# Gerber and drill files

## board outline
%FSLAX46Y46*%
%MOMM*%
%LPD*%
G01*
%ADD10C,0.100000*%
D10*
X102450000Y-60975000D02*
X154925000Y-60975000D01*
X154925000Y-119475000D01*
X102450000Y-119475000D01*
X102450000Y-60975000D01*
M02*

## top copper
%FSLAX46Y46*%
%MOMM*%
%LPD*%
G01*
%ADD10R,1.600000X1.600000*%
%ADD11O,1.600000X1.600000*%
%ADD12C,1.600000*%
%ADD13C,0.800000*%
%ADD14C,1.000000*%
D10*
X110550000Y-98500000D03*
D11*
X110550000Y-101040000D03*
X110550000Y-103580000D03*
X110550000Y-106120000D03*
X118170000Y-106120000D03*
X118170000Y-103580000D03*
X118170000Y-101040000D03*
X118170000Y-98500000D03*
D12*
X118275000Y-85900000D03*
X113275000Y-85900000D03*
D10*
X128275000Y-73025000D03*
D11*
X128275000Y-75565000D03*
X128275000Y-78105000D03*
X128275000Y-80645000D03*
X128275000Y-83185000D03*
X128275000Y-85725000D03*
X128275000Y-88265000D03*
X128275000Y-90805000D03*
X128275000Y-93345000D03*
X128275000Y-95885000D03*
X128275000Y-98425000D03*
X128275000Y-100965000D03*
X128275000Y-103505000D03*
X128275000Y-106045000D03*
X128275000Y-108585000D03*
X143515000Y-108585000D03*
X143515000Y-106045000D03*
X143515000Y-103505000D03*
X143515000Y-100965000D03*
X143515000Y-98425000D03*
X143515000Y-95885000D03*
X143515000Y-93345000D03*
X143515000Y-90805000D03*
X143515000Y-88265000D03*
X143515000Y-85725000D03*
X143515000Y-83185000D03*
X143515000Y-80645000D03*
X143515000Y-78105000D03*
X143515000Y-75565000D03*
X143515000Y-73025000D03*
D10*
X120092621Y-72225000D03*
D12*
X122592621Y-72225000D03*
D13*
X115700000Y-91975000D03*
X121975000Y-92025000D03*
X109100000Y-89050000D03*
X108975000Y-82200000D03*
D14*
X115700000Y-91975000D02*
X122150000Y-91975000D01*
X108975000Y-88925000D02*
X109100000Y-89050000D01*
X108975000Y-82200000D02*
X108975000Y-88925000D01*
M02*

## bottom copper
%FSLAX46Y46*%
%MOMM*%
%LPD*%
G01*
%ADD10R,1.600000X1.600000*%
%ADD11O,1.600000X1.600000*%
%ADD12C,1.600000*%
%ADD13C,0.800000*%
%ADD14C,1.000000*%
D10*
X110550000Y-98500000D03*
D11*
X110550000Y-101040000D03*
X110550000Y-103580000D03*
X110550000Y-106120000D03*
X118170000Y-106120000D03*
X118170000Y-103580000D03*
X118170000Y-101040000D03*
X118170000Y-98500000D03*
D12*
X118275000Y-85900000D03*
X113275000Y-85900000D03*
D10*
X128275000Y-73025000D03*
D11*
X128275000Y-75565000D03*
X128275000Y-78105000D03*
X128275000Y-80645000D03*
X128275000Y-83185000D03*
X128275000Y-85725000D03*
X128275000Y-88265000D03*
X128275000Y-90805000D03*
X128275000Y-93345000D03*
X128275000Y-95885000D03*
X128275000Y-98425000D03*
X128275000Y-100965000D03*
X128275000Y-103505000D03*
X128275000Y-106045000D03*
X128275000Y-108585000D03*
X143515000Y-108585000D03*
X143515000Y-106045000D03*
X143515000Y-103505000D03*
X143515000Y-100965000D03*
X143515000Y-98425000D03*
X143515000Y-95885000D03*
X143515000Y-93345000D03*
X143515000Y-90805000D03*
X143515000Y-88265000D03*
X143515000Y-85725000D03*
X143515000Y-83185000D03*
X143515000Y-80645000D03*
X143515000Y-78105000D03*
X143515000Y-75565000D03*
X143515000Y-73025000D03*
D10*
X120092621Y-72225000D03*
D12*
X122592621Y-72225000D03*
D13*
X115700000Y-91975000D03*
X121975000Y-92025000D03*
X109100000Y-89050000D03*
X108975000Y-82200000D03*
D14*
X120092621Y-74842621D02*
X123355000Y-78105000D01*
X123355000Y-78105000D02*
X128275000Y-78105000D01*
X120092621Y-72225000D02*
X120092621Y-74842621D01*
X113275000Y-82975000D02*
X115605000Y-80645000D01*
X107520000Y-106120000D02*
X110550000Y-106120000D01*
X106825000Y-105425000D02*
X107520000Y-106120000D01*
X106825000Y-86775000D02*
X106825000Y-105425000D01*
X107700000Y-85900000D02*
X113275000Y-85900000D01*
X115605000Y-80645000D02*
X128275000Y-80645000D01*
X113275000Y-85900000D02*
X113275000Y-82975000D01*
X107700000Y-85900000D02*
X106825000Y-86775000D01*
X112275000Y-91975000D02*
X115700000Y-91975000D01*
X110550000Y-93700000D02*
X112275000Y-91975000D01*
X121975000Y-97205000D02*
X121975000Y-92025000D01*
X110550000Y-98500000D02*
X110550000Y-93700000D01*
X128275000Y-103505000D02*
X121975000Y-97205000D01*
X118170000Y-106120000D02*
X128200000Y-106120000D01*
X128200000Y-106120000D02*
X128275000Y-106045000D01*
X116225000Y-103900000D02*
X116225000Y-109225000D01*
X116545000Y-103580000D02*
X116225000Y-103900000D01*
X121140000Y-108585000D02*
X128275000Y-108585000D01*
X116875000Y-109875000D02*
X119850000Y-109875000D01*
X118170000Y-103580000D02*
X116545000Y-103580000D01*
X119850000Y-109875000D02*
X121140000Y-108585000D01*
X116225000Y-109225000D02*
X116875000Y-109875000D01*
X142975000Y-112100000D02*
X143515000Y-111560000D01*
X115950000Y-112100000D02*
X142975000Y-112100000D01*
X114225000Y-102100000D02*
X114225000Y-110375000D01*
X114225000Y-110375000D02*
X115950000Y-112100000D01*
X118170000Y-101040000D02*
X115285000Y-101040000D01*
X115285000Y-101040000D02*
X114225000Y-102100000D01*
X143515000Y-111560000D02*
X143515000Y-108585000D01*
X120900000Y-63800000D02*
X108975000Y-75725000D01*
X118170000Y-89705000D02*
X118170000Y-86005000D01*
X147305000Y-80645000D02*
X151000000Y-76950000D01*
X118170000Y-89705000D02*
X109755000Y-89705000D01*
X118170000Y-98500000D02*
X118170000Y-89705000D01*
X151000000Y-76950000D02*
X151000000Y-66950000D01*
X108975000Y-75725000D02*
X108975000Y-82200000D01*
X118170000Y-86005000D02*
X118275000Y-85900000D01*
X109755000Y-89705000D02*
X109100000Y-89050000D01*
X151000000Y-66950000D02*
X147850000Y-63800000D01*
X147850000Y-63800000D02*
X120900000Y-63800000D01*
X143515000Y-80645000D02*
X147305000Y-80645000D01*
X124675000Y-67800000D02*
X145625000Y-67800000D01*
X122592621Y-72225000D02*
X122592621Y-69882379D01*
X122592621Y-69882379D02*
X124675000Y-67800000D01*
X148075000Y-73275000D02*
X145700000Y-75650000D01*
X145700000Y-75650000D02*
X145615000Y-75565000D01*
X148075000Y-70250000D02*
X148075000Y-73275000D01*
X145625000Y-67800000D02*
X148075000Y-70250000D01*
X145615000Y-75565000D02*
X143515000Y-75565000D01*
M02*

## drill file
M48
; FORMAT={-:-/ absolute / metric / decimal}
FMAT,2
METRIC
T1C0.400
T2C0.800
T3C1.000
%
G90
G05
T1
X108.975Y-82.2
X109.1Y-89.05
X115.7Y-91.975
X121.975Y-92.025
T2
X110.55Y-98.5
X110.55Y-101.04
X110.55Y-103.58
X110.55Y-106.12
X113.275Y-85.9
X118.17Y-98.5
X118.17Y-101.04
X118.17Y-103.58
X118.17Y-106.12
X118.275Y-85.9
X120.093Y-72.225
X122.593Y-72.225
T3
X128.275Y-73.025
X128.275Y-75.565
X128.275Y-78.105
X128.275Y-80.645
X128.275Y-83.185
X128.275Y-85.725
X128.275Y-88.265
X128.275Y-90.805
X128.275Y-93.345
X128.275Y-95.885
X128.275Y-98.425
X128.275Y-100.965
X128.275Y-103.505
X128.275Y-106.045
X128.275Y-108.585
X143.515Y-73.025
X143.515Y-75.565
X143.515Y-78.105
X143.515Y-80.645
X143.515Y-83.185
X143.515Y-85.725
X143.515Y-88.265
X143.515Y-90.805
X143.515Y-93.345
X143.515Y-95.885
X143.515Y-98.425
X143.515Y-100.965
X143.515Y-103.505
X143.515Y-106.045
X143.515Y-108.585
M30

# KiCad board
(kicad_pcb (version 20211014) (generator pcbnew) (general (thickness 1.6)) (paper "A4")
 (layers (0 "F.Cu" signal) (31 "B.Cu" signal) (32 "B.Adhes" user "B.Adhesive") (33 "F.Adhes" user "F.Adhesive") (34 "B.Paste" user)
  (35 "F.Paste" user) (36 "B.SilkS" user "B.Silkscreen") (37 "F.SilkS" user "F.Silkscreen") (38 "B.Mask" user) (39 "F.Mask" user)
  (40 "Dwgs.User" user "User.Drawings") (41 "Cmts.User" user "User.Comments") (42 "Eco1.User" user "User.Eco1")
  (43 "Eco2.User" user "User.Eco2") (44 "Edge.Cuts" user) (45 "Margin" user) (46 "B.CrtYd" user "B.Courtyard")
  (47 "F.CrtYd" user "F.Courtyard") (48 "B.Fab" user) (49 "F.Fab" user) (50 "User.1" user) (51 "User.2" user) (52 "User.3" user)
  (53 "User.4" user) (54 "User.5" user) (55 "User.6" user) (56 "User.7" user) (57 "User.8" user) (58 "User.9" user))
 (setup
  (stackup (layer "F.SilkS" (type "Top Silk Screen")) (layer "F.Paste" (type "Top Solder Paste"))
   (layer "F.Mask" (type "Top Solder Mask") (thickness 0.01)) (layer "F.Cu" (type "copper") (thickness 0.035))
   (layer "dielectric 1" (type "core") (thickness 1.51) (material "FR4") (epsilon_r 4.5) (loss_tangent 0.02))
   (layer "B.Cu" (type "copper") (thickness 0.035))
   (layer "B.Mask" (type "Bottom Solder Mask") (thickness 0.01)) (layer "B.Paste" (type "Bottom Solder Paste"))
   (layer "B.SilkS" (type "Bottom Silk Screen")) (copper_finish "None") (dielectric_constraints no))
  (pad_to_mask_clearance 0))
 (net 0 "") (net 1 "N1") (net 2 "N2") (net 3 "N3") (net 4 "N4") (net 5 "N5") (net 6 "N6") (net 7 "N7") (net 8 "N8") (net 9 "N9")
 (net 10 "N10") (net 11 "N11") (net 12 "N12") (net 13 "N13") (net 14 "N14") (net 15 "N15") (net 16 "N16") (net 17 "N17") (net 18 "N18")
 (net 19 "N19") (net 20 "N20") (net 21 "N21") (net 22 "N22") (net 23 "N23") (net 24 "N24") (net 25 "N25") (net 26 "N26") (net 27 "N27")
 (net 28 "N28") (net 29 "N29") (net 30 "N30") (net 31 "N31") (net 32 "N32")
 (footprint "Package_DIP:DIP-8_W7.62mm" (layer "F.Cu") (at 110.55 98.5)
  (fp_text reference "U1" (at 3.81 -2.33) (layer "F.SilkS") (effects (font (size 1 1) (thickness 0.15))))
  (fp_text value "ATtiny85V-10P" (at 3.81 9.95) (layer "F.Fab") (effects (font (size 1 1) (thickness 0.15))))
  (pad "1" thru_hole rect (at 0 0) (size 1.6 1.6) (drill 0.8) (layers *.Cu *.Mask) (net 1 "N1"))
  (pad "2" thru_hole oval (at 0 2.54) (size 1.6 1.6) (drill 0.8) (layers *.Cu *.Mask) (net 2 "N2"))
  (pad "3" thru_hole oval (at 0 5.08) (size 1.6 1.6) (drill 0.8) (layers *.Cu *.Mask) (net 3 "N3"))
  (pad "4" thru_hole oval (at 0 7.62) (size 1.6 1.6) (drill 0.8) (layers *.Cu *.Mask) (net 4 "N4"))
  (pad "5" thru_hole oval (at 7.62 7.62) (size 1.6 1.6) (drill 0.8) (layers *.Cu *.Mask) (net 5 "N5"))
  (pad "6" thru_hole oval (at 7.62 5.08) (size 1.6 1.6) (drill 0.8) (layers *.Cu *.Mask) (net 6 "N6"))
  (pad "7" thru_hole oval (at 7.62 2.54) (size 1.6 1.6) (drill 0.8) (layers *.Cu *.Mask) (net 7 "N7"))
  (pad "8" thru_hole oval (at 7.62 0) (size 1.6 1.6) (drill 0.8) (layers *.Cu *.Mask) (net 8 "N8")))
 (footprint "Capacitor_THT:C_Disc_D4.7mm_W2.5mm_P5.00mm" (layer "F.Cu") (at 118.275 85.9 180)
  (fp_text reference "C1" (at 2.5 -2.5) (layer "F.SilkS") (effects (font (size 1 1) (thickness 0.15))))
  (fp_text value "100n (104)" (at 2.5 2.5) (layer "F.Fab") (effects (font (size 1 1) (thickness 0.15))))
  (pad "1" thru_hole circle (at 0 0 180) (size 1.6 1.6) (drill 0.8) (layers *.Cu *.Mask) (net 8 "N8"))
  (pad "2" thru_hole circle (at 5 0 180) (size 1.6 1.6) (drill 0.8) (layers *.Cu *.Mask) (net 4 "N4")))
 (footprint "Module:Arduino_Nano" (layer "F.Cu") (at 128.275 73.025)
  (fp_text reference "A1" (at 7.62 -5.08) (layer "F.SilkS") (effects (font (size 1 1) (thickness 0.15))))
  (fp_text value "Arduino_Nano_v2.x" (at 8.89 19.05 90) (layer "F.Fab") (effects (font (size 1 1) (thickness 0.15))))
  (pad "1" thru_hole rect (at 0 0) (size 1.6 1.6) (drill 1) (layers *.Cu *.Mask) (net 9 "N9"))
  (pad "2" thru_hole oval (at 0 2.54) (size 1.6 1.6) (drill 1) (layers *.Cu *.Mask) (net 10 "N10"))
  (pad "3" thru_hole oval (at 0 5.08) (size 1.6 1.6) (drill 1) (layers *.Cu *.Mask) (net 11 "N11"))
  (pad "4" thru_hole oval (at 0 7.62) (size 1.6 1.6) (drill 1) (layers *.Cu *.Mask) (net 4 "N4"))
  (pad "5" thru_hole oval (at 0 10.16) (size 1.6 1.6) (drill 1) (layers *.Cu *.Mask) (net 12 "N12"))
  (pad "6" thru_hole oval (at 0 12.7) (size 1.6 1.6) (drill 1) (layers *.Cu *.Mask) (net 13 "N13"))
  (pad "7" thru_hole oval (at 0 15.24) (size 1.6 1.6) (drill 1) (layers *.Cu *.Mask) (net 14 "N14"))
  (pad "8" thru_hole oval (at 0 17.78) (size 1.6 1.6) (drill 1) (layers *.Cu *.Mask) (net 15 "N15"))
  (pad "9" thru_hole oval (at 0 20.32) (size 1.6 1.6) (drill 1) (layers *.Cu *.Mask) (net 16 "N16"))
  (pad "10" thru_hole oval (at 0 22.86) (size 1.6 1.6) (drill 1) (layers *.Cu *.Mask) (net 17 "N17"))
  (pad "11" thru_hole oval (at 0 25.4) (size 1.6 1.6) (drill 1) (layers *.Cu *.Mask) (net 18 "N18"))
  (pad "12" thru_hole oval (at 0 27.94) (size 1.6 1.6) (drill 1) (layers *.Cu *.Mask) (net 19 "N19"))
  (pad "13" thru_hole oval (at 0 30.48) (size 1.6 1.6) (drill 1) (layers *.Cu *.Mask) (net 1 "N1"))
  (pad "14" thru_hole oval (at 0 33.02) (size 1.6 1.6) (drill 1) (layers *.Cu *.Mask) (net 5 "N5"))
  (pad "15" thru_hole oval (at 0 35.56) (size 1.6 1.6) (drill 1) (layers *.Cu *.Mask) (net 6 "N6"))
  (pad "16" thru_hole oval (at 15.24 35.56) (size 1.6 1.6) (drill 1) (layers *.Cu *.Mask) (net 7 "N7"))
  (pad "17" thru_hole oval (at 15.24 33.02) (size 1.6 1.6) (drill 1) (layers *.Cu *.Mask) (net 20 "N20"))
  (pad "18" thru_hole oval (at 15.24 30.48) (size 1.6 1.6) (drill 1) (layers *.Cu *.Mask) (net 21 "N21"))
  (pad "19" thru_hole oval (at 15.24 27.94) (size 1.6 1.6) (drill 1) (layers *.Cu *.Mask) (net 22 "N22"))
  (pad "20" thru_hole oval (at 15.24 25.4) (size 1.6 1.6) (drill 1) (layers *.Cu *.Mask) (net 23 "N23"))
  (pad "21" thru_hole oval (at 15.24 22.86) (size 1.6 1.6) (drill 1) (layers *.Cu *.Mask) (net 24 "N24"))
  (pad "22" thru_hole oval (at 15.24 20.32) (size 1.6 1.6) (drill 1) (layers *.Cu *.Mask) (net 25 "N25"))
  (pad "23" thru_hole oval (at 15.24 17.78) (size 1.6 1.6) (drill 1) (layers *.Cu *.Mask) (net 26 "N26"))
  (pad "24" thru_hole oval (at 15.24 15.24) (size 1.6 1.6) (drill 1) (layers *.Cu *.Mask) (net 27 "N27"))
  (pad "25" thru_hole oval (at 15.24 12.7) (size 1.6 1.6) (drill 1) (layers *.Cu *.Mask) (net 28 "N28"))
  (pad "26" thru_hole oval (at 15.24 10.16) (size 1.6 1.6) (drill 1) (layers *.Cu *.Mask) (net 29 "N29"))
  (pad "27" thru_hole oval (at 15.24 7.62) (size 1.6 1.6) (drill 1) (layers *.Cu *.Mask) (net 8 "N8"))
  (pad "28" thru_hole oval (at 15.24 5.08) (size 1.6 1.6) (drill 1) (layers *.Cu *.Mask) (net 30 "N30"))
  (pad "29" thru_hole oval (at 15.24 2.54) (size 1.6 1.6) (drill 1) (layers *.Cu *.Mask) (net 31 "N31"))
  (pad "30" thru_hole oval (at 15.24 0) (size 1.6 1.6) (drill 1) (layers *.Cu *.Mask) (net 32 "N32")))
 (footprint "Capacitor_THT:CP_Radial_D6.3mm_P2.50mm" (layer "F.Cu") (at 120.092621 72.225)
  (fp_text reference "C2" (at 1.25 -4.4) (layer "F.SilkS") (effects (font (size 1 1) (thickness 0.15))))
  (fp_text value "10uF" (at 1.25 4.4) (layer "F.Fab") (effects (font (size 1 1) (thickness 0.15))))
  (pad "1" thru_hole rect (at 0 0) (size 1.6 1.6) (drill 0.8) (layers *.Cu *.Mask) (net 11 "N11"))
  (pad "2" thru_hole circle (at 2.5 0) (size 1.6 1.6) (drill 0.8) (layers *.Cu *.Mask) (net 31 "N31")))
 (gr_rect (start 102.45 60.975) (end 154.925 119.475) (layer "Edge.Cuts") (width 0.1) (fill none))
 (segment (start 120.092621 74.842621) (end 123.355 78.105) (width 1) (layer "B.Cu") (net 11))
 (segment (start 123.355 78.105) (end 128.275 78.105) (width 1) (layer "B.Cu") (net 11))
 (segment (start 120.092621 72.225) (end 120.092621 74.842621) (width 1) (layer "B.Cu") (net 11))
 (segment (start 113.275 82.975) (end 115.605 80.645) (width 1) (layer "B.Cu") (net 4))
 (segment (start 107.52 106.12) (end 110.55 106.12) (width 1) (layer "B.Cu") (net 4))
 (segment (start 106.825 105.425) (end 107.52 106.12) (width 1) (layer "B.Cu") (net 4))
 (segment (start 106.825 86.775) (end 106.825 105.425) (width 1) (layer "B.Cu") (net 4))
 (segment (start 107.7 85.9) (end 113.275 85.9) (width 1) (layer "B.Cu") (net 4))
 (segment (start 115.605 80.645) (end 128.275 80.645) (width 1) (layer "B.Cu") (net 4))
 (segment (start 113.275 85.9) (end 113.275 82.975) (width 1) (layer "B.Cu") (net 4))
 (segment (start 107.7 85.9) (end 106.825 86.775) (width 1) (layer "B.Cu") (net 4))
 (segment (start 115.7 91.975) (end 122.15 91.975) (width 1) (layer "F.Cu") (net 1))
 (via (at 115.7 91.975) (size 0.8) (drill 0.4) (layers "F.Cu" "B.Cu") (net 1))
 (via (at 121.975 92.025) (size 0.8) (drill 0.4) (layers "F.Cu" "B.Cu") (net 1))
 (segment (start 112.275 91.975) (end 115.7 91.975) (width 1) (layer "B.Cu") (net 1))
 (segment (start 110.55 93.7) (end 112.275 91.975) (width 1) (layer "B.Cu") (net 1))
 (segment (start 121.975 97.205) (end 121.975 92.025) (width 1) (layer "B.Cu") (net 1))
 (segment (start 110.55 98.5) (end 110.55 93.7) (width 1) (layer "B.Cu") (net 1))
 (segment (start 128.275 103.505) (end 121.975 97.205) (width 1) (layer "B.Cu") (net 1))
 (segment (start 118.17 106.12) (end 128.2 106.12) (width 1) (layer "B.Cu") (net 5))
 (segment (start 128.2 106.12) (end 128.275 106.045) (width 1) (layer "B.Cu") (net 5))
 (segment (start 116.225 103.9) (end 116.225 109.225) (width 1) (layer "B.Cu") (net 6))
 (segment (start 116.545 103.58) (end 116.225 103.9) (width 1) (layer "B.Cu") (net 6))
 (segment (start 121.14 108.585) (end 128.275 108.585) (width 1) (layer "B.Cu") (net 6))
 (segment (start 116.875 109.875) (end 119.85 109.875) (width 1) (layer "B.Cu") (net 6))
 (segment (start 118.17 103.58) (end 116.545 103.58) (width 1) (layer "B.Cu") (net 6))
 (segment (start 119.85 109.875) (end 121.14 108.585) (width 1) (layer "B.Cu") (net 6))
 (segment (start 116.225 109.225) (end 116.875 109.875) (width 1) (layer "B.Cu") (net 6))
 (segment (start 142.975 112.1) (end 143.515 111.56) (width 1) (layer "B.Cu") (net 7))
 (segment (start 115.95 112.1) (end 142.975 112.1) (width 1) (layer "B.Cu") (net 7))
 (segment (start 114.225 102.1) (end 114.225 110.375) (width 1) (layer "B.Cu") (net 7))
 (segment (start 114.225 110.375) (end 115.95 112.1) (width 1) (layer "B.Cu") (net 7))
 (segment (start 118.17 101.04) (end 115.285 101.04) (width 1) (layer "B.Cu") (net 7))
 (segment (start 115.285 101.04) (end 114.225 102.1) (width 1) (layer "B.Cu") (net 7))
 (segment (start 143.515 111.56) (end 143.515 108.585) (width 1) (layer "B.Cu") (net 7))
 (segment (start 108.975 88.925) (end 109.1 89.05) (width 1) (layer "F.Cu") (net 8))
 (segment (start 108.975 82.2) (end 108.975 88.925) (width 1) (layer "F.Cu") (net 8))
 (via (at 109.1 89.05) (size 0.8) (drill 0.4) (layers "F.Cu" "B.Cu") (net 8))
 (via (at 108.975 82.2) (size 0.8) (drill 0.4) (layers "F.Cu" "B.Cu") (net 8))
 (segment (start 120.9 63.8) (end 108.975 75.725) (width 1) (layer "B.Cu") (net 8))
 (segment (start 118.17 89.705) (end 118.17 86.005) (width 1) (layer "B.Cu") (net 8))
 (segment (start 147.305 80.645) (end 151 76.95) (width 1) (layer "B.Cu") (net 8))
 (segment (start 118.17 89.705) (end 109.755 89.705) (width 1) (layer "B.Cu") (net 8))
 (segment (start 118.17 98.5) (end 118.17 89.705) (width 1) (layer "B.Cu") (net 8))
 (segment (start 151 76.95) (end 151 66.95) (width 1) (layer "B.Cu") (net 8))
 (segment (start 108.975 75.725) (end 108.975 82.2) (width 1) (layer "B.Cu") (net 8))
 (segment (start 118.17 86.005) (end 118.275 85.9) (width 1) (layer "B.Cu") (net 8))
 (segment (start 109.755 89.705) (end 109.1 89.05) (width 1) (layer "B.Cu") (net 8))
 (segment (start 151 66.95) (end 147.85 63.8) (width 1) (layer "B.Cu") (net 8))
 (segment (start 147.85 63.8) (end 120.9 63.8) (width 1) (layer "B.Cu") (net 8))
 (segment (start 143.515 80.645) (end 147.305 80.645) (width 1) (layer "B.Cu") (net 8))
 (segment (start 124.675 67.8) (end 145.625 67.8) (width 1) (layer "B.Cu") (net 31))
 (segment (start 122.592621 72.225) (end 122.592621 69.882379) (width 1) (layer "B.Cu") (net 31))
 (segment (start 122.592621 69.882379) (end 124.675 67.8) (width 1) (layer "B.Cu") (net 31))
 (segment (start 148.075 73.275) (end 145.7 75.65) (width 1) (layer "B.Cu") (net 31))
 (segment (start 145.7 75.65) (end 145.615 75.565) (width 1) (layer "B.Cu") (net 31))
 (segment (start 148.075 70.25) (end 148.075 73.275) (width 1) (layer "B.Cu") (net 31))
 (segment (start 145.625 67.8) (end 148.075 70.25) (width 1) (layer "B.Cu") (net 31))
 (segment (start 145.615 75.565) (end 143.515 75.565) (width 1) (layer "B.Cu") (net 31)))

